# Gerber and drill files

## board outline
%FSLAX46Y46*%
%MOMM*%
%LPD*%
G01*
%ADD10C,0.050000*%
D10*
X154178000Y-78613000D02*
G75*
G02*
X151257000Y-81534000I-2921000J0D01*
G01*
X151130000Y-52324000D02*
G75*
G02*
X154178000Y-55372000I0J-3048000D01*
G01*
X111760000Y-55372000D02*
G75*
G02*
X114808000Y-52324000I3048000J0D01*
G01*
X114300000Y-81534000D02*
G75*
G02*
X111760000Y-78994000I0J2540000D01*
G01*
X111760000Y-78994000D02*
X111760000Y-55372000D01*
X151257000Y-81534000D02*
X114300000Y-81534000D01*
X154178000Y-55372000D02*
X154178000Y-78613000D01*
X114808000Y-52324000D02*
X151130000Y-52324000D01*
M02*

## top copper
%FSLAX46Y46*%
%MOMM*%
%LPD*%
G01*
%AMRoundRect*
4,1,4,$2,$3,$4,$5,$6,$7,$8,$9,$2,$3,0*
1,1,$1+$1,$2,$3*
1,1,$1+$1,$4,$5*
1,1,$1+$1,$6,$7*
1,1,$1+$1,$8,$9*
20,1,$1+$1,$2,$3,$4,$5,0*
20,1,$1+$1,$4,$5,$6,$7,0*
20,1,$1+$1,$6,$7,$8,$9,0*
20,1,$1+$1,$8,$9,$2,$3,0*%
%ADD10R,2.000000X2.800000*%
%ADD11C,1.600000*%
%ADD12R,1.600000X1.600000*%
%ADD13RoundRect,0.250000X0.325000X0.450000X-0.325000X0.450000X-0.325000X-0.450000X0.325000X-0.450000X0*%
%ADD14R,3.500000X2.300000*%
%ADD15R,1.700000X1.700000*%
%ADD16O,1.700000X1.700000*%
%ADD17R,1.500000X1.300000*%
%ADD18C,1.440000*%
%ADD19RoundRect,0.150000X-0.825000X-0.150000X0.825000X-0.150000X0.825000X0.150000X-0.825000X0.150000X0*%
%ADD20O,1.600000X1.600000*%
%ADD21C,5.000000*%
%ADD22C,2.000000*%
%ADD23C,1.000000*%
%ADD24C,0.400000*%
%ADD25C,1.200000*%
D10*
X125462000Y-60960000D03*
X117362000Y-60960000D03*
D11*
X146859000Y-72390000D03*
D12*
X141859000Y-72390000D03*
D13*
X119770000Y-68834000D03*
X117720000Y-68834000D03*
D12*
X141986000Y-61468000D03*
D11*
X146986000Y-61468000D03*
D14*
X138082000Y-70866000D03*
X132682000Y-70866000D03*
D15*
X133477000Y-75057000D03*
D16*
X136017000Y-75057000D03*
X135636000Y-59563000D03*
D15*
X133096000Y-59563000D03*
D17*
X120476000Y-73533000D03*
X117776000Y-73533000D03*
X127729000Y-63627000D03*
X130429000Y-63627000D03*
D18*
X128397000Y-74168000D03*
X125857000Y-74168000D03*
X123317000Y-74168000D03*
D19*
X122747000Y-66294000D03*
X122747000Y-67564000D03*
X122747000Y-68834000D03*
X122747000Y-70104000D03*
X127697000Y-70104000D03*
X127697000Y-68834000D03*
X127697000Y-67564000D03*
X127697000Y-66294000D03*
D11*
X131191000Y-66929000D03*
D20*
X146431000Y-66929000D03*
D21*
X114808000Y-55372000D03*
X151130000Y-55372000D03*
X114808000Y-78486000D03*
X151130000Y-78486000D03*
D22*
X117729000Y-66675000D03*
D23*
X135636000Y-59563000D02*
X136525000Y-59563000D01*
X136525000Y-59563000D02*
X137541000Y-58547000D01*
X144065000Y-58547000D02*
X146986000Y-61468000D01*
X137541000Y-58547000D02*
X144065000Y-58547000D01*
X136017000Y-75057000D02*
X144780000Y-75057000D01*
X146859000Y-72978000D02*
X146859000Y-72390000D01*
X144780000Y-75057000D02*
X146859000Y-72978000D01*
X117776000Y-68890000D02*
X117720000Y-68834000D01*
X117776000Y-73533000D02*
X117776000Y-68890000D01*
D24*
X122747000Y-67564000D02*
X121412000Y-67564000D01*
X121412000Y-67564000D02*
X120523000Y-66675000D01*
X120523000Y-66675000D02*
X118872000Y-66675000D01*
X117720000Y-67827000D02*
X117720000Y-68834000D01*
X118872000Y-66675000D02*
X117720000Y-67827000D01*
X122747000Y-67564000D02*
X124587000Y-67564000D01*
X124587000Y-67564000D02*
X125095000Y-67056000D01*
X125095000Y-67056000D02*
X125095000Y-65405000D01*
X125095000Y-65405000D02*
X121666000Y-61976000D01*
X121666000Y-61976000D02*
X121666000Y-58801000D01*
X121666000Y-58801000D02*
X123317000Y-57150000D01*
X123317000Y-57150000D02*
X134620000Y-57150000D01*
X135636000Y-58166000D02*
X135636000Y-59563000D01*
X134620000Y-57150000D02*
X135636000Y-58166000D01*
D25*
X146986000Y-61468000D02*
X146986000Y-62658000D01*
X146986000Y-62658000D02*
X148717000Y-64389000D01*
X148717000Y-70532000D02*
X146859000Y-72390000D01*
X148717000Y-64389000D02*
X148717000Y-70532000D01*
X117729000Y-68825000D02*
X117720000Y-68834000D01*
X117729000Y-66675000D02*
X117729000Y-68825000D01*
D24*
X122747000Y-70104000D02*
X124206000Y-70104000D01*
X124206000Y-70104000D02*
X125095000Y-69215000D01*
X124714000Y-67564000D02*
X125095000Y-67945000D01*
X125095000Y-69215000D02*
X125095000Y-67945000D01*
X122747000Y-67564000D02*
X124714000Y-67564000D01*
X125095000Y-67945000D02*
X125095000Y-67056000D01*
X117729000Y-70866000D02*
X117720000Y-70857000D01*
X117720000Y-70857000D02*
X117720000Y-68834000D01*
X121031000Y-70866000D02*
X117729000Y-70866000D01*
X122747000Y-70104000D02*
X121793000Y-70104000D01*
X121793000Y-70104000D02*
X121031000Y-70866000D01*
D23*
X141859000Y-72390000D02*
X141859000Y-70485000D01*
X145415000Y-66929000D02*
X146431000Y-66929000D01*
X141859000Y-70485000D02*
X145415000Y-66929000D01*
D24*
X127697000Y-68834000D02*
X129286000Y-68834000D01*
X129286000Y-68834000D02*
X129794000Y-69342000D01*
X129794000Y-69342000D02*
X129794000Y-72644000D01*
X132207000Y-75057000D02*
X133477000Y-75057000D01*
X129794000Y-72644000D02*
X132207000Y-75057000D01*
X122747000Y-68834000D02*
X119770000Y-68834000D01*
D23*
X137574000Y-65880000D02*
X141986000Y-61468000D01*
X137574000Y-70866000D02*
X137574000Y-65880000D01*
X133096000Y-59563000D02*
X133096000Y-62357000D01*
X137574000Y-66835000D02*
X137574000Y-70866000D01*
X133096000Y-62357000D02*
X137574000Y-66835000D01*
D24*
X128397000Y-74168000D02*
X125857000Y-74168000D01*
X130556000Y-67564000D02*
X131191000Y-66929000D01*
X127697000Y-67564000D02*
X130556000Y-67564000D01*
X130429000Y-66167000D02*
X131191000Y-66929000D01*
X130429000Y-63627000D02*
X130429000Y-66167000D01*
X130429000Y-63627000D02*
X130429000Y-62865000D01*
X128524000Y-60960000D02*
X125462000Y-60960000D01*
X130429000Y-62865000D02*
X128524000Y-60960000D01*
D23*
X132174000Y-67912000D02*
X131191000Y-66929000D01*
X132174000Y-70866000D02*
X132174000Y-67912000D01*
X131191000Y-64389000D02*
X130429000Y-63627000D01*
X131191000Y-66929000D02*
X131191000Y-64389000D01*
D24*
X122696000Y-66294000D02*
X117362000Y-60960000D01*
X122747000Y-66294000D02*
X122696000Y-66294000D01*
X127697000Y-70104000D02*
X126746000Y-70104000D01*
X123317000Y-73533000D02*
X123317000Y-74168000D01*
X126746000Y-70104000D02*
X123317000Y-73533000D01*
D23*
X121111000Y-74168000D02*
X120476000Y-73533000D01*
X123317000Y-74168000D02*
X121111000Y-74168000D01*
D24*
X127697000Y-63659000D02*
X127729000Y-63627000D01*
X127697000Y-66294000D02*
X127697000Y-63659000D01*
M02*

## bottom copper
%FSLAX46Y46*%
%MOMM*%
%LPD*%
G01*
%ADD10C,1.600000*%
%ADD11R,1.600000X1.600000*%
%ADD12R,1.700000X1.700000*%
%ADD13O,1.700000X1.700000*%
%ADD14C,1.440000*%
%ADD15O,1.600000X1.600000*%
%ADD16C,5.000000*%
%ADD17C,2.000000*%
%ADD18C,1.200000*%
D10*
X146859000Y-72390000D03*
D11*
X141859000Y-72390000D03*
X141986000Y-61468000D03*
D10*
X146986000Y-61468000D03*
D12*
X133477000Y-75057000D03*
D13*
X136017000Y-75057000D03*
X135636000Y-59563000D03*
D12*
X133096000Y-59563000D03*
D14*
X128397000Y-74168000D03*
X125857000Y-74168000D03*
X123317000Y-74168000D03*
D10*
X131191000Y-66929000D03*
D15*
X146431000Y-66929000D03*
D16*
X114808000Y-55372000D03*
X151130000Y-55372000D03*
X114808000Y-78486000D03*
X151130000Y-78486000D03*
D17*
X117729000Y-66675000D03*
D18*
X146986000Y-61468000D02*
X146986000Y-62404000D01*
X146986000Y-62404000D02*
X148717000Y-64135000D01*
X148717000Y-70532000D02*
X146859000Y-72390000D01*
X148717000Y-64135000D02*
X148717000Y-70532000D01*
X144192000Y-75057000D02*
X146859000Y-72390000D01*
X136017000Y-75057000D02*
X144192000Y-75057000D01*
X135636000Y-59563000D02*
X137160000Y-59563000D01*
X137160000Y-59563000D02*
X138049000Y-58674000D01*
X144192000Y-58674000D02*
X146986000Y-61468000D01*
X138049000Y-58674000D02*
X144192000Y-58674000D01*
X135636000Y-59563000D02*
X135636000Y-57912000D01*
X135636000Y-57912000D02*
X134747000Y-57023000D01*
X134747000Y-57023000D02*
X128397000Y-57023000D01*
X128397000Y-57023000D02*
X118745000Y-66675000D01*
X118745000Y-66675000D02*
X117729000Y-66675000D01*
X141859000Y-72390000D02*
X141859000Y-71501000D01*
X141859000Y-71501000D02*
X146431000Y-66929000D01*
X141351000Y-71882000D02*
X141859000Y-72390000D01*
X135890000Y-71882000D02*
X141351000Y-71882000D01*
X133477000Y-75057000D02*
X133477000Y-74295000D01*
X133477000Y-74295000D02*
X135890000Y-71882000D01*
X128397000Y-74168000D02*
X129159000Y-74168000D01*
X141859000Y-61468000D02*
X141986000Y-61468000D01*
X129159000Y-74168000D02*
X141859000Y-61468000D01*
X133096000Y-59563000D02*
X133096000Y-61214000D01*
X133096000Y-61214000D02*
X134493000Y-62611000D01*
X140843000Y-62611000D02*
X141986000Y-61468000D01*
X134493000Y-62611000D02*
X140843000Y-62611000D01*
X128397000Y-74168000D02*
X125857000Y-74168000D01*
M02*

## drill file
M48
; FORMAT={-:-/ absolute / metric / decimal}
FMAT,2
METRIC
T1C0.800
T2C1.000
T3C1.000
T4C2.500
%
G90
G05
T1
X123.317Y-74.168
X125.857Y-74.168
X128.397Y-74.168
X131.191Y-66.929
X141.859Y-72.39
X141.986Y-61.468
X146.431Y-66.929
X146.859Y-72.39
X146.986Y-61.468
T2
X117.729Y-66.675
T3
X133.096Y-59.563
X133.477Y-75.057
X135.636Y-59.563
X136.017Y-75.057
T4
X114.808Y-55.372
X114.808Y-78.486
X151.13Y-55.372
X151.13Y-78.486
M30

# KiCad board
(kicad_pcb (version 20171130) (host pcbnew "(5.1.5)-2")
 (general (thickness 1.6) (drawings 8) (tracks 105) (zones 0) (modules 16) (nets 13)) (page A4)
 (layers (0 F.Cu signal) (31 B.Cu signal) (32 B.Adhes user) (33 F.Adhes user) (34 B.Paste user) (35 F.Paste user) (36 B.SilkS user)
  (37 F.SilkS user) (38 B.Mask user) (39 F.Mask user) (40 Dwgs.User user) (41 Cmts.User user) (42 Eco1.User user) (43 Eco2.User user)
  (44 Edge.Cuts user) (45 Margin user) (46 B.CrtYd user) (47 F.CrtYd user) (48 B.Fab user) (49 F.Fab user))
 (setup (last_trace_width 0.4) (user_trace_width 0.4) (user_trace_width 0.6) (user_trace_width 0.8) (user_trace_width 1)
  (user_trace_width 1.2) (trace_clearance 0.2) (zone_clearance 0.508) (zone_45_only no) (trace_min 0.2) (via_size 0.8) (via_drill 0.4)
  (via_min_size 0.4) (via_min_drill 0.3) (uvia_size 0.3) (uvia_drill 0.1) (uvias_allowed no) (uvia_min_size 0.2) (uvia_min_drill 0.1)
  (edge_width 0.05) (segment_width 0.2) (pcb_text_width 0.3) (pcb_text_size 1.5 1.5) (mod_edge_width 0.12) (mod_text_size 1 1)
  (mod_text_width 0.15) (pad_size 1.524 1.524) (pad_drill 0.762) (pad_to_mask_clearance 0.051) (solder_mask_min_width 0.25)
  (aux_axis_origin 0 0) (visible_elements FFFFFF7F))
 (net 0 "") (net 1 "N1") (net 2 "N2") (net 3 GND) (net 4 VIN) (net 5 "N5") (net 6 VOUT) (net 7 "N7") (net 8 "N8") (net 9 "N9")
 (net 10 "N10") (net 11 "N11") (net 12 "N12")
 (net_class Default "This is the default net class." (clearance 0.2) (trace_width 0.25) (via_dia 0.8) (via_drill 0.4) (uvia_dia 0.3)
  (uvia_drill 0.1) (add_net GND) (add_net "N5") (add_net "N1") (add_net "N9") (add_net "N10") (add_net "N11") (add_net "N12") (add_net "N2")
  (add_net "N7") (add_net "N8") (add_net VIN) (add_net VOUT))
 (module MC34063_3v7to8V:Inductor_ (layer F.Cu) (at 121.412 60.96)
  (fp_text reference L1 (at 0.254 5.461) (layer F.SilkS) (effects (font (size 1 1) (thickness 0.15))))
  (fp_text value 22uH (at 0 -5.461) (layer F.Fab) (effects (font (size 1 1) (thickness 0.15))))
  (pad 2 smd rect (at 4.05 0) (size 2 2.8) (layers F.Cu F.Paste F.Mask) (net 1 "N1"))
  (pad 1 smd rect (at -4.05 0) (size 2 2.8) (layers F.Cu F.Paste F.Mask) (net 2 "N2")))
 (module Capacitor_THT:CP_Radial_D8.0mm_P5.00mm (layer F.Cu) (at 141.859 72.39)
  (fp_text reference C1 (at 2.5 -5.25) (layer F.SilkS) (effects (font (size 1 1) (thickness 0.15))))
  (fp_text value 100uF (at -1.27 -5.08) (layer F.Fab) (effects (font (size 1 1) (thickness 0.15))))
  (pad 2 thru_hole circle (at 5 0) (size 1.6 1.6) (drill 0.8) (layers *.Cu *.Mask) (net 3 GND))
  (pad 1 thru_hole rect (at 0 0) (size 1.6 1.6) (drill 0.8) (layers *.Cu *.Mask) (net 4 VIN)))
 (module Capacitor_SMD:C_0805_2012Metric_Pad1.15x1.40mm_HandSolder (layer F.Cu) (at 118.745 68.834 180)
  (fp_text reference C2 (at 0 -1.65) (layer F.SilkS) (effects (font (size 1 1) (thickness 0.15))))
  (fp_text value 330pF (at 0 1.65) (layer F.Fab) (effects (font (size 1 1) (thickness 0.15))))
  (pad 1 smd roundrect (at -1.025 0 180) (size 1.15 1.4) (layers F.Cu F.Paste F.Mask) (roundrect_rratio 0.217391) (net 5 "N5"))
  (pad 2 smd roundrect (at 1.025 0 180) (size 1.15 1.4) (layers F.Cu F.Paste F.Mask) (roundrect_rratio 0.217391) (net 3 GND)))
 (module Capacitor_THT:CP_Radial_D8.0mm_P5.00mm (layer F.Cu) (at 141.986 61.468)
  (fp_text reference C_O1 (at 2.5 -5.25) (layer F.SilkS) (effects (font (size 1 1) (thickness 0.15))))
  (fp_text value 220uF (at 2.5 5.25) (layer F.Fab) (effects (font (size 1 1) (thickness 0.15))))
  (pad 1 thru_hole rect (at 0 0) (size 1.6 1.6) (drill 0.8) (layers *.Cu *.Mask) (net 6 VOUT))
  (pad 2 thru_hole circle (at 5 0) (size 1.6 1.6) (drill 0.8) (layers *.Cu *.Mask) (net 3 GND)))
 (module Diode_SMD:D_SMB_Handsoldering (layer F.Cu) (at 135.382 70.866 180)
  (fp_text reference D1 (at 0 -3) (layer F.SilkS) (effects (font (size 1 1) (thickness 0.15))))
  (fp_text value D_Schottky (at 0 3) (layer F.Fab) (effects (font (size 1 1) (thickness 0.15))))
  (pad 1 smd rect (at -2.7 0 180) (size 3.5 2.3) (layers F.Cu F.Paste F.Mask) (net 6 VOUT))
  (pad 2 smd rect (at 2.7 0 180) (size 3.5 2.3) (layers F.Cu F.Paste F.Mask) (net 1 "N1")))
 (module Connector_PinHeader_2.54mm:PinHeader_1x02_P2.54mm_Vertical (layer F.Cu) (at 133.477 75.057 90)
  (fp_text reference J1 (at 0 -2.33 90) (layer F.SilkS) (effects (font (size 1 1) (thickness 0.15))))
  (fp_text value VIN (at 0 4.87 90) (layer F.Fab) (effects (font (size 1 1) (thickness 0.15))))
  (pad 1 thru_hole rect (at 0 0 90) (size 1.7 1.7) (drill 1) (layers *.Cu *.Mask) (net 4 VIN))
  (pad 2 thru_hole oval (at 0 2.54 90) (size 1.7 1.7) (drill 1) (layers *.Cu *.Mask) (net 3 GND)))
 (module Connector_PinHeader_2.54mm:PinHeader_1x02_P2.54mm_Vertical (layer F.Cu) (at 133.096 59.563 90)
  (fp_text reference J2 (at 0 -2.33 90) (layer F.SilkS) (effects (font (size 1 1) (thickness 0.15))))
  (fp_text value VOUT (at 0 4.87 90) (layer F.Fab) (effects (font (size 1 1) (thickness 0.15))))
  (pad 2 thru_hole oval (at 0 2.54 90) (size 1.7 1.7) (drill 1) (layers *.Cu *.Mask) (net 3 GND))
  (pad 1 thru_hole rect (at 0 0 90) (size 1.7 1.7) (drill 1) (layers *.Cu *.Mask) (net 6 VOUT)))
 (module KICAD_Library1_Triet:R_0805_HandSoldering (layer F.Cu) (at 119.126 73.533 180)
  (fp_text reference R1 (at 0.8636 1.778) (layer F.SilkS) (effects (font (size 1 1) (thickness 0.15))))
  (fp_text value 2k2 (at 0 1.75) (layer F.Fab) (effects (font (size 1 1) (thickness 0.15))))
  (pad 1 smd rect (at -1.35 0 180) (size 1.5 1.3) (layers F.Cu F.Paste F.Mask) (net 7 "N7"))
  (pad 2 smd rect (at 1.35 0 180) (size 1.5 1.3) (layers F.Cu F.Paste F.Mask) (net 3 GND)))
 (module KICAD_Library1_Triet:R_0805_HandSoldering (layer F.Cu) (at 129.079 63.627 180)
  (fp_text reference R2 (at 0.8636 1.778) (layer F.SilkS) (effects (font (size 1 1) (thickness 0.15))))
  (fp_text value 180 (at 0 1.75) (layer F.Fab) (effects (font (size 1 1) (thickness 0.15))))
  (pad 2 smd rect (at 1.35 0 180) (size 1.5 1.3) (layers F.Cu F.Paste F.Mask) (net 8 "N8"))
  (pad 1 smd rect (at -1.35 0 180) (size 1.5 1.3) (layers F.Cu F.Paste F.Mask) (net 1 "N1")))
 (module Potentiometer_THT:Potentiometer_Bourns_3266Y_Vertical (layer F.Cu) (at 128.397 74.168)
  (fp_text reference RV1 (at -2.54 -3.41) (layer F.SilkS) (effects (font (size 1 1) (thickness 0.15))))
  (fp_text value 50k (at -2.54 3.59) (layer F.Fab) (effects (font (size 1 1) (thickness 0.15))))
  (pad 1 thru_hole circle (at 0 0) (size 1.44 1.44) (drill 0.8) (layers *.Cu *.Mask) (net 6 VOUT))
  (pad 2 thru_hole circle (at -2.54 0) (size 1.44 1.44) (drill 0.8) (layers *.Cu *.Mask) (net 6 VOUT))
  (pad 3 thru_hole circle (at -5.08 0) (size 1.44 1.44) (drill 0.8) (layers *.Cu *.Mask) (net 7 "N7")))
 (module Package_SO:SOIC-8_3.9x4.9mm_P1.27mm (layer F.Cu) (at 125.222 68.199)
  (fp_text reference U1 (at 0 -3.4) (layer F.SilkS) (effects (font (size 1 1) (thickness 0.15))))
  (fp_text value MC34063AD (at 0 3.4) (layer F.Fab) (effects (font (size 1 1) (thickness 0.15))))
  (pad 1 smd roundrect (at -2.475 -1.905) (size 1.95 0.6) (layers F.Cu F.Paste F.Mask) (roundrect_rratio 0.25) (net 2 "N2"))
  (pad 2 smd roundrect (at -2.475 -0.635) (size 1.95 0.6) (layers F.Cu F.Paste F.Mask) (roundrect_rratio 0.25) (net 3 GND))
  (pad 3 smd roundrect (at -2.475 0.635) (size 1.95 0.6) (layers F.Cu F.Paste F.Mask) (roundrect_rratio 0.25) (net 5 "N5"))
  (pad 4 smd roundrect (at -2.475 1.905) (size 1.95 0.6) (layers F.Cu F.Paste F.Mask) (roundrect_rratio 0.25) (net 3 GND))
  (pad 5 smd roundrect (at 2.475 1.905) (size 1.95 0.6) (layers F.Cu F.Paste F.Mask) (roundrect_rratio 0.25) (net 7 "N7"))
  (pad 6 smd roundrect (at 2.475 0.635) (size 1.95 0.6) (layers F.Cu F.Paste F.Mask) (roundrect_rratio 0.25) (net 4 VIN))
  (pad 7 smd roundrect (at 2.475 -0.635) (size 1.95 0.6) (layers F.Cu F.Paste F.Mask) (roundrect_rratio 0.25) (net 1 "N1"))
  (pad 8 smd roundrect (at 2.475 -1.905) (size 1.95 0.6) (layers F.Cu F.Paste F.Mask) (roundrect_rratio 0.25) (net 8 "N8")))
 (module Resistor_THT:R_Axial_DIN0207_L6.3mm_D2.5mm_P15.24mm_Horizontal (layer F.Cu) (at 131.191 66.929)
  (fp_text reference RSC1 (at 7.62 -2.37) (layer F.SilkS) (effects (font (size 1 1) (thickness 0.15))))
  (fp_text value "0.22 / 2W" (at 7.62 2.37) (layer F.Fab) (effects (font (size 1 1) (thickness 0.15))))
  (pad 1 thru_hole circle (at 0 0) (size 1.6 1.6) (drill 0.8) (layers *.Cu *.Mask) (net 1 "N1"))
  (pad 2 thru_hole oval (at 15.24 0) (size 1.6 1.6) (drill 0.8) (layers *.Cu *.Mask) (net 4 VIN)))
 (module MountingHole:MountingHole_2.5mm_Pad (layer F.Cu) (at 114.808 55.372)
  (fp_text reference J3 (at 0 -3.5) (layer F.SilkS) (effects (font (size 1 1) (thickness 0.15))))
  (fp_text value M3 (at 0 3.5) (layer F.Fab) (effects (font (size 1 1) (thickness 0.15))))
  (pad 1 thru_hole circle (at 0 0) (size 5 5) (drill 2.5) (layers *.Cu *.Mask) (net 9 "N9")))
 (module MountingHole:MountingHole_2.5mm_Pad (layer F.Cu) (at 151.13 55.372)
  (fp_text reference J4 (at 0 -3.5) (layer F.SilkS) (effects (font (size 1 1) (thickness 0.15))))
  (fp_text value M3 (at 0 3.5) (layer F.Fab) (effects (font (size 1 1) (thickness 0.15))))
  (pad 1 thru_hole circle (at 0 0) (size 5 5) (drill 2.5) (layers *.Cu *.Mask) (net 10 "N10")))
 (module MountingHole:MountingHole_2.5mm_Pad (layer F.Cu) (at 114.808 78.486)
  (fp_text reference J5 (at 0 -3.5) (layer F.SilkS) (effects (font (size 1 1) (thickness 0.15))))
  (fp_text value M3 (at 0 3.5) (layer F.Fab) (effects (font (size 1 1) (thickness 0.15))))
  (pad 1 thru_hole circle (at 0 0) (size 5 5) (drill 2.5) (layers *.Cu *.Mask) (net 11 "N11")))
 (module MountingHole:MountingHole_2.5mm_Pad (layer F.Cu) (at 151.13 78.486)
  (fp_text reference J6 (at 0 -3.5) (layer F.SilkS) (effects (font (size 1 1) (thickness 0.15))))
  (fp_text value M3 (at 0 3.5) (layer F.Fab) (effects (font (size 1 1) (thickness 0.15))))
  (pad 1 thru_hole circle (at 0 0) (size 5 5) (drill 2.5) (layers *.Cu *.Mask) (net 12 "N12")))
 (gr_arc (start 151.257 78.613) (end 151.257 81.534) (angle -90) (layer Edge.Cuts) (width 0.05))
 (gr_arc (start 151.13 55.372) (end 154.178 55.372) (angle -90) (layer Edge.Cuts) (width 0.05))
 (gr_arc (start 114.808 55.372) (end 114.808 52.324) (angle -90) (layer Edge.Cuts) (width 0.05))
 (gr_arc (start 114.3 78.994) (end 111.76 78.994) (angle -90) (layer Edge.Cuts) (width 0.05))
 (gr_line (start 111.76 78.994) (end 111.76 55.372) (layer Edge.Cuts) (width 0.05))
 (gr_line (start 151.257 81.534) (end 114.3 81.534) (layer Edge.Cuts) (width 0.05))
 (gr_line (start 154.178 55.372) (end 154.178 78.613) (layer Edge.Cuts) (width 0.05))
 (gr_line (start 114.808 52.324) (end 151.13 52.324) (layer Edge.Cuts) (width 0.05))
 (segment (start 135.636 59.563) (end 136.525 59.563) (width 1) (layer F.Cu) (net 3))
 (segment (start 136.525 59.563) (end 137.541 58.547) (width 1) (layer F.Cu) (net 3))
 (segment (start 144.065 58.547) (end 146.986 61.468) (width 1) (layer F.Cu) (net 3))
 (segment (start 137.541 58.547) (end 144.065 58.547) (width 1) (layer F.Cu) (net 3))
 (segment (start 136.017 75.057) (end 144.78 75.057) (width 1) (layer F.Cu) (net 3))
 (segment (start 146.859 72.978) (end 146.859 72.39) (width 1) (layer F.Cu) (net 3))
 (segment (start 144.78 75.057) (end 146.859 72.978) (width 1) (layer F.Cu) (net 3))
 (segment (start 117.776 68.89) (end 117.72 68.834) (width 1) (layer F.Cu) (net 3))
 (segment (start 117.776 73.533) (end 117.776 68.89) (width 1) (layer F.Cu) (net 3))
 (segment (start 122.747 67.564) (end 121.412 67.564) (width 0.4) (layer F.Cu) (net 3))
 (segment (start 121.412 67.564) (end 120.523 66.675) (width 0.4) (layer F.Cu) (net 3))
 (segment (start 120.523 66.675) (end 118.872 66.675) (width 0.4) (layer F.Cu) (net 3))
 (segment (start 117.72 67.827) (end 117.72 68.834) (width 0.4) (layer F.Cu) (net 3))
 (segment (start 118.872 66.675) (end 117.72 67.827) (width 0.4) (layer F.Cu) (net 3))
 (segment (start 122.747 67.564) (end 124.587 67.564) (width 0.4) (layer F.Cu) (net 3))
 (segment (start 124.587 67.564) (end 125.095 67.056) (width 0.4) (layer F.Cu) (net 3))
 (segment (start 125.095 67.056) (end 125.095 65.405) (width 0.4) (layer F.Cu) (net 3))
 (segment (start 125.095 65.405) (end 121.666 61.976) (width 0.4) (layer F.Cu) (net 3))
 (segment (start 121.666 61.976) (end 121.666 58.801) (width 0.4) (layer F.Cu) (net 3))
 (segment (start 121.666 58.801) (end 123.317 57.15) (width 0.4) (layer F.Cu) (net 3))
 (segment (start 123.317 57.15) (end 134.62 57.15) (width 0.4) (layer F.Cu) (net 3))
 (segment (start 135.636 58.166) (end 135.636 59.563) (width 0.4) (layer F.Cu) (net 3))
 (segment (start 134.62 57.15) (end 135.636 58.166) (width 0.4) (layer F.Cu) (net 3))
 (segment (start 146.986 61.468) (end 146.986 62.658) (width 1.2) (layer F.Cu) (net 3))
 (segment (start 146.986 62.658) (end 148.717 64.389) (width 1.2) (layer F.Cu) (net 3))
 (segment (start 148.717 70.532) (end 146.859 72.39) (width 1.2) (layer F.Cu) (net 3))
 (segment (start 148.717 64.389) (end 148.717 70.532) (width 1.2) (layer F.Cu) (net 3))
 (segment (start 146.986 61.468) (end 146.986 62.404) (width 1.2) (layer B.Cu) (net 3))
 (segment (start 146.986 62.404) (end 148.717 64.135) (width 1.2) (layer B.Cu) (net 3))
 (segment (start 148.717 70.532) (end 146.859 72.39) (width 1.2) (layer B.Cu) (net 3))
 (segment (start 148.717 64.135) (end 148.717 70.532) (width 1.2) (layer B.Cu) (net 3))
 (segment (start 144.192 75.057) (end 146.859 72.39) (width 1.2) (layer B.Cu) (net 3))
 (segment (start 136.017 75.057) (end 144.192 75.057) (width 1.2) (layer B.Cu) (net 3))
 (segment (start 135.636 59.563) (end 137.16 59.563) (width 1.2) (layer B.Cu) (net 3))
 (segment (start 137.16 59.563) (end 138.049 58.674) (width 1.2) (layer B.Cu) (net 3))
 (segment (start 144.192 58.674) (end 146.986 61.468) (width 1.2) (layer B.Cu) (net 3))
 (segment (start 138.049 58.674) (end 144.192 58.674) (width 1.2) (layer B.Cu) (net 3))
 (segment (start 135.636 59.563) (end 135.636 57.912) (width 1.2) (layer B.Cu) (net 3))
 (segment (start 135.636 57.912) (end 134.747 57.023) (width 1.2) (layer B.Cu) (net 3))
 (segment (start 134.747 57.023) (end 128.397 57.023) (width 1.2) (layer B.Cu) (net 3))
 (segment (start 128.397 57.023) (end 118.745 66.675) (width 1.2) (layer B.Cu) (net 3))
 (via (at 117.729 66.675) (size 2) (drill 1) (layers F.Cu B.Cu) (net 3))
 (segment (start 118.745 66.675) (end 117.729 66.675) (width 1.2) (layer B.Cu) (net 3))
 (segment (start 117.729 68.825) (end 117.72 68.834) (width 1.2) (layer F.Cu) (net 3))
 (segment (start 117.729 66.675) (end 117.729 68.825) (width 1.2) (layer F.Cu) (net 3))
 (segment (start 122.747 70.104) (end 124.206 70.104) (width 0.4) (layer F.Cu) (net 3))
 (segment (start 124.206 70.104) (end 125.095 69.215) (width 0.4) (layer F.Cu) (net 3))
 (segment (start 124.714 67.564) (end 125.095 67.945) (width 0.4) (layer F.Cu) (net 3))
 (segment (start 125.095 69.215) (end 125.095 67.945) (width 0.4) (layer F.Cu) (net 3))
 (segment (start 122.747 67.564) (end 124.714 67.564) (width 0.4) (layer F.Cu) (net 3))
 (segment (start 125.095 67.945) (end 125.095 67.056) (width 0.4) (layer F.Cu) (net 3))
 (segment (start 117.729 70.866) (end 117.72 70.857) (width 0.4) (layer F.Cu) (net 3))
 (segment (start 117.72 70.857) (end 117.72 68.834) (width 0.4) (layer F.Cu) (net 3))
 (segment (start 121.031 70.866) (end 117.729 70.866) (width 0.4) (layer F.Cu) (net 3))
 (segment (start 122.747 70.104) (end 121.793 70.104) (width 0.4) (layer F.Cu) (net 3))
 (segment (start 121.793 70.104) (end 121.031 70.866) (width 0.4) (layer F.Cu) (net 3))
 (segment (start 141.859 72.39) (end 141.859 70.485) (width 1) (layer F.Cu) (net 4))
 (segment (start 145.415 66.929) (end 146.431 66.929) (width 1) (layer F.Cu) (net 4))
 (segment (start 141.859 70.485) (end 145.415 66.929) (width 1) (layer F.Cu) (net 4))
 (segment (start 127.697 68.834) (end 129.286 68.834) (width 0.4) (layer F.Cu) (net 4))
 (segment (start 129.286 68.834) (end 129.794 69.342) (width 0.4) (layer F.Cu) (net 4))
 (segment (start 129.794 69.342) (end 129.794 72.644) (width 0.4) (layer F.Cu) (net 4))
 (segment (start 132.207 75.057) (end 133.477 75.057) (width 0.4) (layer F.Cu) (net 4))
 (segment (start 129.794 72.644) (end 132.207 75.057) (width 0.4) (layer F.Cu) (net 4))
 (segment (start 141.859 72.39) (end 141.859 71.501) (width 1.2) (layer B.Cu) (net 4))
 (segment (start 141.859 71.501) (end 146.431 66.929) (width 1.2) (layer B.Cu) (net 4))
 (segment (start 141.351 71.882) (end 141.859 72.39) (width 1.2) (layer B.Cu) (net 4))
 (segment (start 135.89 71.882) (end 141.351 71.882) (width 1.2) (layer B.Cu) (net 4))
 (segment (start 133.477 75.057) (end 133.477 74.295) (width 1.2) (layer B.Cu) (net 4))
 (segment (start 133.477 74.295) (end 135.89 71.882) (width 1.2) (layer B.Cu) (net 4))
 (segment (start 122.747 68.834) (end 119.77 68.834) (width 0.4) (layer F.Cu) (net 5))
 (segment (start 137.574 65.88) (end 141.986 61.468) (width 1) (layer F.Cu) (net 6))
 (segment (start 137.574 70.866) (end 137.574 65.88) (width 1) (layer F.Cu) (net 6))
 (segment (start 133.096 59.563) (end 133.096 62.357) (width 1) (layer F.Cu) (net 6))
 (segment (start 137.574 66.835) (end 137.574 70.866) (width 1) (layer F.Cu) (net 6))
 (segment (start 133.096 62.357) (end 137.574 66.835) (width 1) (layer F.Cu) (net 6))
 (segment (start 128.397 74.168) (end 125.857 74.168) (width 0.4) (layer F.Cu) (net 6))
 (segment (start 128.397 74.168) (end 129.159 74.168) (width 1.2) (layer B.Cu) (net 6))
 (segment (start 141.859 61.468) (end 141.986 61.468) (width 1.2) (layer B.Cu) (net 6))
 (segment (start 129.159 74.168) (end 141.859 61.468) (width 1.2) (layer B.Cu) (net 6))
 (segment (start 133.096 59.563) (end 133.096 61.214) (width 1.2) (layer B.Cu) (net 6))
 (segment (start 133.096 61.214) (end 134.493 62.611) (width 1.2) (layer B.Cu) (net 6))
 (segment (start 140.843 62.611) (end 141.986 61.468) (width 1.2) (layer B.Cu) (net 6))
 (segment (start 134.493 62.611) (end 140.843 62.611) (width 1.2) (layer B.Cu) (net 6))
 (segment (start 128.397 74.168) (end 125.857 74.168) (width 1.2) (layer B.Cu) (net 6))
 (segment (start 130.556 67.564) (end 131.191 66.929) (width 0.4) (layer F.Cu) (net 1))
 (segment (start 127.697 67.564) (end 130.556 67.564) (width 0.4) (layer F.Cu) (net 1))
 (segment (start 130.429 66.167) (end 131.191 66.929) (width 0.4) (layer F.Cu) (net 1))
 (segment (start 130.429 63.627) (end 130.429 66.167) (width 0.4) (layer F.Cu) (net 1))
 (segment (start 130.429 63.627) (end 130.429 62.865) (width 0.4) (layer F.Cu) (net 1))
 (segment (start 128.524 60.96) (end 125.462 60.96) (width 0.4) (layer F.Cu) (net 1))
 (segment (start 130.429 62.865) (end 128.524 60.96) (width 0.4) (layer F.Cu) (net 1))
 (segment (start 132.174 67.912) (end 131.191 66.929) (width 1) (layer F.Cu) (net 1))
 (segment (start 132.174 70.866) (end 132.174 67.912) (width 1) (layer F.Cu) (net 1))
 (segment (start 131.191 64.389) (end 130.429 63.627) (width 1) (layer F.Cu) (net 1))
 (segment (start 131.191 66.929) (end 131.191 64.389) (width 1) (layer F.Cu) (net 1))
 (segment (start 122.696 66.294) (end 117.362 60.96) (width 0.4) (layer F.Cu) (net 2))
 (segment (start 122.747 66.294) (end 122.696 66.294) (width 0.4) (layer F.Cu) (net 2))
 (segment (start 127.697 70.104) (end 126.746 70.104) (width 0.4) (layer F.Cu) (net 7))
 (segment (start 123.317 73.533) (end 123.317 74.168) (width 0.4) (layer F.Cu) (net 7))
 (segment (start 126.746 70.104) (end 123.317 73.533) (width 0.4) (layer F.Cu) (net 7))
 (segment (start 121.111 74.168) (end 120.476 73.533) (width 1) (layer F.Cu) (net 7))
 (segment (start 123.317 74.168) (end 121.111 74.168) (width 1) (layer F.Cu) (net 7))
 (segment (start 127.697 63.659) (end 127.729 63.627) (width 0.4) (layer F.Cu) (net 8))
 (segment (start 127.697 66.294) (end 127.697 63.659) (width 0.4) (layer F.Cu) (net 8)))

